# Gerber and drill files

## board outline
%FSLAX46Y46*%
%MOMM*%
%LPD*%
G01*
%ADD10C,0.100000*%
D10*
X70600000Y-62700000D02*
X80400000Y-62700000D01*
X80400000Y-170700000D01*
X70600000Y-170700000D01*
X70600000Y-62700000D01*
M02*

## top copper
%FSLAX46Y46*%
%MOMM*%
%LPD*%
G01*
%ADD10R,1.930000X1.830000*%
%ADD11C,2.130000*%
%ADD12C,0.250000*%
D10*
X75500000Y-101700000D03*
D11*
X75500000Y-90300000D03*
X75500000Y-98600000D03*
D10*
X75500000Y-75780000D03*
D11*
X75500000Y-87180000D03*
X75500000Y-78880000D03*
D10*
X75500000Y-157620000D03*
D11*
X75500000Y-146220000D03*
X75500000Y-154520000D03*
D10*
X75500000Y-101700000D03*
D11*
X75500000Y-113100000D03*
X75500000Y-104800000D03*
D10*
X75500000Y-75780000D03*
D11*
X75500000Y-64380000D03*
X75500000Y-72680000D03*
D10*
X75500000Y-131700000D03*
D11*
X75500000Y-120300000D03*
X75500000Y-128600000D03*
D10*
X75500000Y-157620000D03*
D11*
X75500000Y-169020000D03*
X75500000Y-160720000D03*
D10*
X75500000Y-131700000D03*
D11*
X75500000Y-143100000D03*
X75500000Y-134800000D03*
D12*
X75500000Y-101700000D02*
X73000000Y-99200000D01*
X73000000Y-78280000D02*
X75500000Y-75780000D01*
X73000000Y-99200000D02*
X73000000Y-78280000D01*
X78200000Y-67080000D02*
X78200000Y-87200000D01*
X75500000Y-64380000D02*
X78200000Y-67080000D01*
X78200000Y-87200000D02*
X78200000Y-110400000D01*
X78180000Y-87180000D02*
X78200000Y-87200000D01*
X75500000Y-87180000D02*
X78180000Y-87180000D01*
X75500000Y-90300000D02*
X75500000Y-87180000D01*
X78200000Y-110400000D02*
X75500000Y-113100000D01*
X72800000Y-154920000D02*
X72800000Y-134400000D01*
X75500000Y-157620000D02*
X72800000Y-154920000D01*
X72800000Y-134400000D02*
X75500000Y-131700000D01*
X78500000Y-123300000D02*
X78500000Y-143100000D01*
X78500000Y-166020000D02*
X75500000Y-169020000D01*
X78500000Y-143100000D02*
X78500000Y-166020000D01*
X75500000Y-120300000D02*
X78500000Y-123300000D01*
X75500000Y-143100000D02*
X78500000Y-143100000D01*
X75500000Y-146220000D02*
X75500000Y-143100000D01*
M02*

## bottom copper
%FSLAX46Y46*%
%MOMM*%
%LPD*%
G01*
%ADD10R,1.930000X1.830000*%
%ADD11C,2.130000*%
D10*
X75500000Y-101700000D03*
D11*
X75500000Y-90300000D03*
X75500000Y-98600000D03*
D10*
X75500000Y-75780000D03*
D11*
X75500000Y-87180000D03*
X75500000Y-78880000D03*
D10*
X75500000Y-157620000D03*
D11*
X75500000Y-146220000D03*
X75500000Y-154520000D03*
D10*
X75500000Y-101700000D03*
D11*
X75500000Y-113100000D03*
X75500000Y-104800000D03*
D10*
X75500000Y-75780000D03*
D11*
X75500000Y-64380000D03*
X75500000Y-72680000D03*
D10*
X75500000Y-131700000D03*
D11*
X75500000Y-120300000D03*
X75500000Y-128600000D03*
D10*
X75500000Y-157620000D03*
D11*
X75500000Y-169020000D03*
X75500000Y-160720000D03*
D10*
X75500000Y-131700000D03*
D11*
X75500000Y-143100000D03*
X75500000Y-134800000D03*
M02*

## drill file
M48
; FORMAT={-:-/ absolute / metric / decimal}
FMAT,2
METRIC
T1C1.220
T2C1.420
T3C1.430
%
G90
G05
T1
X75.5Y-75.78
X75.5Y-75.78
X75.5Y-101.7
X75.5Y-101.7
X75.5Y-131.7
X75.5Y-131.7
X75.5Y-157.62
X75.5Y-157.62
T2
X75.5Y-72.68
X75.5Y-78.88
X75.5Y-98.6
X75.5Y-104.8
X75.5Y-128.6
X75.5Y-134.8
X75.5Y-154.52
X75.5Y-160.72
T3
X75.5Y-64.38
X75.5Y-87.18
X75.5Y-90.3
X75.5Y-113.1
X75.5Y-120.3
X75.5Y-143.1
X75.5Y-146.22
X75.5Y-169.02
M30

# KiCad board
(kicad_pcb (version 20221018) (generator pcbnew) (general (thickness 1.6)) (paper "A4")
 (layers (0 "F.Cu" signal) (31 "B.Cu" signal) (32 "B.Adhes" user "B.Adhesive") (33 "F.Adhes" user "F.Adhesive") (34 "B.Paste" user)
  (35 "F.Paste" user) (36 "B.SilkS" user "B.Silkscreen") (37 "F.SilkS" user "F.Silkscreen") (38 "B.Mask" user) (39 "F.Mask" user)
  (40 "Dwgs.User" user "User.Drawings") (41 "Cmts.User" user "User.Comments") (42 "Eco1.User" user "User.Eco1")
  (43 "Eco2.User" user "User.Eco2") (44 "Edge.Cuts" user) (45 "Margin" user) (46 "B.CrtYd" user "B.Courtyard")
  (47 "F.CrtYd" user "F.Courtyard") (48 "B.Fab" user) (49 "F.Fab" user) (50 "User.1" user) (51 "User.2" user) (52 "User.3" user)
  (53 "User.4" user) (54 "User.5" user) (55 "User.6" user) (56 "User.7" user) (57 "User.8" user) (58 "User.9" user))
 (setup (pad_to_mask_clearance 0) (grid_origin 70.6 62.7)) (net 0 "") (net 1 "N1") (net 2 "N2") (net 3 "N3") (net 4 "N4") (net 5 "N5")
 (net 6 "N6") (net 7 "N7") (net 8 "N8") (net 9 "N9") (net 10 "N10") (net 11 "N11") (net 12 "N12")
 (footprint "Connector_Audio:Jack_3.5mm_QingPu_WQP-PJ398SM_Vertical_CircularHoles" (layer "F.Cu") (at 75.5 101.7 180)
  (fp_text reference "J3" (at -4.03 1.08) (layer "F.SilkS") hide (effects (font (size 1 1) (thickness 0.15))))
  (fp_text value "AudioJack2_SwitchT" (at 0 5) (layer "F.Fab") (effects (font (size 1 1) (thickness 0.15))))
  (pad "S" thru_hole rect (at 0 0) (size 1.93 1.83) (drill 1.22) (layers "*.Cu" "*.Mask") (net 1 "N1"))
  (pad "T" thru_hole circle (at 0 11.4) (size 2.13 2.13) (drill 1.43) (layers "*.Cu" "*.Mask") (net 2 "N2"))
  (pad "TN" thru_hole circle (at 0 3.1) (size 2.13 2.13) (drill 1.42) (layers "*.Cu" "*.Mask") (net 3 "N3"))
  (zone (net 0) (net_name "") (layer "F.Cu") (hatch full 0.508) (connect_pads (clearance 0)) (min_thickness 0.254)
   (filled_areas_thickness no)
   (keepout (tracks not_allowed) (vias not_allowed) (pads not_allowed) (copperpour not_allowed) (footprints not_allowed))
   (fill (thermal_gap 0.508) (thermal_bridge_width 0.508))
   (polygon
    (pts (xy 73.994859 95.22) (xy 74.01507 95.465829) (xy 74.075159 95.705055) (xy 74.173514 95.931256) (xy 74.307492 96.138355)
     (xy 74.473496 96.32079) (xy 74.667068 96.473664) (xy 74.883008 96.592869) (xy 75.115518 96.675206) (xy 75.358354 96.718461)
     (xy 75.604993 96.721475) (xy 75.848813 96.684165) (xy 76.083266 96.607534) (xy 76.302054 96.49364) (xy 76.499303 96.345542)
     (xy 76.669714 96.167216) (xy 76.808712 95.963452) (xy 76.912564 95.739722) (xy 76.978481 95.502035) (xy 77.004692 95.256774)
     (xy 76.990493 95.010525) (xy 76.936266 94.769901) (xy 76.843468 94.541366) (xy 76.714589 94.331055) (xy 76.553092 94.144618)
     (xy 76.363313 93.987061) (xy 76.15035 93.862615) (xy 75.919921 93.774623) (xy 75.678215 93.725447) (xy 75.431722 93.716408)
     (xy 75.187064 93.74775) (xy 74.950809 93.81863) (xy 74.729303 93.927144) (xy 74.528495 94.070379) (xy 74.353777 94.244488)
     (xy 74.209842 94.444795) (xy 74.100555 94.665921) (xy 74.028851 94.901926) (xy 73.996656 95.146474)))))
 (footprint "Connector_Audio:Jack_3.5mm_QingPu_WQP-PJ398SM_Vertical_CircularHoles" (layer "F.Cu") (at 75.5 75.78)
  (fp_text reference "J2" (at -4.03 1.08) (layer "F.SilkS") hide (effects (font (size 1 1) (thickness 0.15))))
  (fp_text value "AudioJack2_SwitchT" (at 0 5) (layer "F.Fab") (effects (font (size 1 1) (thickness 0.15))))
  (pad "S" thru_hole rect (at 0 0 180) (size 1.93 1.83) (drill 1.22) (layers "*.Cu" "*.Mask") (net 1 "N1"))
  (pad "T" thru_hole circle (at 0 11.4 180) (size 2.13 2.13) (drill 1.43) (layers "*.Cu" "*.Mask") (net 2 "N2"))
  (pad "TN" thru_hole circle (at 0 3.1 180) (size 2.13 2.13) (drill 1.42) (layers "*.Cu" "*.Mask") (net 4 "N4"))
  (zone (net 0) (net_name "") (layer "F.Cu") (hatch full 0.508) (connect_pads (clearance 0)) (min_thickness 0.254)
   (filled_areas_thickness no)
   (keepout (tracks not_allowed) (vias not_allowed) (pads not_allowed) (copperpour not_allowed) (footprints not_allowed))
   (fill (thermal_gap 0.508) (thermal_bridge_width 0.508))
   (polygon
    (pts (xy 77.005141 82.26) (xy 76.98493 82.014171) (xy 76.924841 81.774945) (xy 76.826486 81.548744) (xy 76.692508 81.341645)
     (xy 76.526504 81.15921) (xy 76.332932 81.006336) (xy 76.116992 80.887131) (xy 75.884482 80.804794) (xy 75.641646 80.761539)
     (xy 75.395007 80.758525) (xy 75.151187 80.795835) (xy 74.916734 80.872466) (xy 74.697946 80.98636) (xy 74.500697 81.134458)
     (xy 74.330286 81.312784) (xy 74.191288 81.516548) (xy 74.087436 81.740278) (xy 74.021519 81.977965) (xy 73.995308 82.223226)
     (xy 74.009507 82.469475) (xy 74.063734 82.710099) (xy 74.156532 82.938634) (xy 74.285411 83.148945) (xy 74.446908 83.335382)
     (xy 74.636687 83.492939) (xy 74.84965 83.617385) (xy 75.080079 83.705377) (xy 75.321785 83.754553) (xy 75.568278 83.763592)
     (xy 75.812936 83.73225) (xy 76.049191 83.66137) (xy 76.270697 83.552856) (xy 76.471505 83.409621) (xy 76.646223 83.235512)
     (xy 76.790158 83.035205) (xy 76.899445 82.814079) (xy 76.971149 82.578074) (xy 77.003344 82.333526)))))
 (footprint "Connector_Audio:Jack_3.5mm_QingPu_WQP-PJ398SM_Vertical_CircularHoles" (layer "F.Cu") (at 75.5 157.62 180)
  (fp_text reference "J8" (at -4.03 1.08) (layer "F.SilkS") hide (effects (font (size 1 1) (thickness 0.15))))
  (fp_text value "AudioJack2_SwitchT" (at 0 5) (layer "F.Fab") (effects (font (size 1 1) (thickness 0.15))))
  (pad "S" thru_hole rect (at 0 0) (size 1.93 1.83) (drill 1.22) (layers "*.Cu" "*.Mask") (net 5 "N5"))
  (pad "T" thru_hole circle (at 0 11.4) (size 2.13 2.13) (drill 1.43) (layers "*.Cu" "*.Mask") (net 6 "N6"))
  (pad "TN" thru_hole circle (at 0 3.1) (size 2.13 2.13) (drill 1.42) (layers "*.Cu" "*.Mask") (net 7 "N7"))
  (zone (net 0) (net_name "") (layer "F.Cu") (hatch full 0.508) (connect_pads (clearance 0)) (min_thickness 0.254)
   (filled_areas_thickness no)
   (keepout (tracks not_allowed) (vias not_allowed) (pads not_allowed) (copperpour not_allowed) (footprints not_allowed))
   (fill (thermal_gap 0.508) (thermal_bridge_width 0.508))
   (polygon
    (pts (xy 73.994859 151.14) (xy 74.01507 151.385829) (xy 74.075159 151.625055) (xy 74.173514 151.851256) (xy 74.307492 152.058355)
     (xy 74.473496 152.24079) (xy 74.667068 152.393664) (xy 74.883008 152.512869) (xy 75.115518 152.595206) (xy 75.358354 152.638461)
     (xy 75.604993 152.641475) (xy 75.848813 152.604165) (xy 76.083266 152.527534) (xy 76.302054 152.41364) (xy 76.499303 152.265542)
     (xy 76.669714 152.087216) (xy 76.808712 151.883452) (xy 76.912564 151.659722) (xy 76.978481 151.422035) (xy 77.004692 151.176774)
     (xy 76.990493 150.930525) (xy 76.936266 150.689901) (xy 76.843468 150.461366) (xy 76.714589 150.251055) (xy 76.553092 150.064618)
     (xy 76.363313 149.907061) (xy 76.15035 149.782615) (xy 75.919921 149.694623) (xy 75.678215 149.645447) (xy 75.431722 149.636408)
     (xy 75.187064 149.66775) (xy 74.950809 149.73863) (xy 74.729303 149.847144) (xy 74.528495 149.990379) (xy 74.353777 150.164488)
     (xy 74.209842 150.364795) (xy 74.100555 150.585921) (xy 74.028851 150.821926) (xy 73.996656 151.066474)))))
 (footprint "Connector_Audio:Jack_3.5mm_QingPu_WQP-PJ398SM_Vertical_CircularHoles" (layer "F.Cu") (at 75.5 101.7)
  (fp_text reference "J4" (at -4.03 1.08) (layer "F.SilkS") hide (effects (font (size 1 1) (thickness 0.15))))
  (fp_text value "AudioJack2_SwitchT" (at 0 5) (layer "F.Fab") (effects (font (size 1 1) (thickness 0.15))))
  (pad "S" thru_hole rect (at 0 0 180) (size 1.93 1.83) (drill 1.22) (layers "*.Cu" "*.Mask") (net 1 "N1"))
  (pad "T" thru_hole circle (at 0 11.4 180) (size 2.13 2.13) (drill 1.43) (layers "*.Cu" "*.Mask") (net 2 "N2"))
  (pad "TN" thru_hole circle (at 0 3.1 180) (size 2.13 2.13) (drill 1.42) (layers "*.Cu" "*.Mask") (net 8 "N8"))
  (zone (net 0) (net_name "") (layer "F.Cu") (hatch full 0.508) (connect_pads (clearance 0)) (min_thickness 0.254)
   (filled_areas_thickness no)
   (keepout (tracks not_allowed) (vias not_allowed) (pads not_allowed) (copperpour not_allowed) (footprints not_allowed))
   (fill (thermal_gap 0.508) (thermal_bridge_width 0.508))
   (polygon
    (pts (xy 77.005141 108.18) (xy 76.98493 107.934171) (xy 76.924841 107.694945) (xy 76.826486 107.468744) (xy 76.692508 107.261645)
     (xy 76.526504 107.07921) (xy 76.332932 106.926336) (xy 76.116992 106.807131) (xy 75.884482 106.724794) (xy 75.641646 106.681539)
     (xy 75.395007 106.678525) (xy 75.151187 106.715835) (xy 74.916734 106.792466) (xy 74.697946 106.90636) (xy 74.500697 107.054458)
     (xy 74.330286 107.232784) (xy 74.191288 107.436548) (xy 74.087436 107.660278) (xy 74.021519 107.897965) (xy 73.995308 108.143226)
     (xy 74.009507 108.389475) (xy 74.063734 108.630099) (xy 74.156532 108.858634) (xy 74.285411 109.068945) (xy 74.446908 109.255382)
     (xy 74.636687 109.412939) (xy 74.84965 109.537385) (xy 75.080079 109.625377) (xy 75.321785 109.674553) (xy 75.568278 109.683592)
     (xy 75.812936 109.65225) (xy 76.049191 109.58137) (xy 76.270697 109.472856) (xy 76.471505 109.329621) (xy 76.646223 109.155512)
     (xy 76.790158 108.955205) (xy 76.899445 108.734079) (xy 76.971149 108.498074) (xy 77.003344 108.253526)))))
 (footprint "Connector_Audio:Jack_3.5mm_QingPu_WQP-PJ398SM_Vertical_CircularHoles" (layer "F.Cu") (at 75.5 75.78 180)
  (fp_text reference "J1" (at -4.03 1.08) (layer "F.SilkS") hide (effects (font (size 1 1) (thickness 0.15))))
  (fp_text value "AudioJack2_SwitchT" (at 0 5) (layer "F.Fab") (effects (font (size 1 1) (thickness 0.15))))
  (pad "S" thru_hole rect (at 0 0) (size 1.93 1.83) (drill 1.22) (layers "*.Cu" "*.Mask") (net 1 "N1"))
  (pad "T" thru_hole circle (at 0 11.4) (size 2.13 2.13) (drill 1.43) (layers "*.Cu" "*.Mask") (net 2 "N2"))
  (pad "TN" thru_hole circle (at 0 3.1) (size 2.13 2.13) (drill 1.42) (layers "*.Cu" "*.Mask") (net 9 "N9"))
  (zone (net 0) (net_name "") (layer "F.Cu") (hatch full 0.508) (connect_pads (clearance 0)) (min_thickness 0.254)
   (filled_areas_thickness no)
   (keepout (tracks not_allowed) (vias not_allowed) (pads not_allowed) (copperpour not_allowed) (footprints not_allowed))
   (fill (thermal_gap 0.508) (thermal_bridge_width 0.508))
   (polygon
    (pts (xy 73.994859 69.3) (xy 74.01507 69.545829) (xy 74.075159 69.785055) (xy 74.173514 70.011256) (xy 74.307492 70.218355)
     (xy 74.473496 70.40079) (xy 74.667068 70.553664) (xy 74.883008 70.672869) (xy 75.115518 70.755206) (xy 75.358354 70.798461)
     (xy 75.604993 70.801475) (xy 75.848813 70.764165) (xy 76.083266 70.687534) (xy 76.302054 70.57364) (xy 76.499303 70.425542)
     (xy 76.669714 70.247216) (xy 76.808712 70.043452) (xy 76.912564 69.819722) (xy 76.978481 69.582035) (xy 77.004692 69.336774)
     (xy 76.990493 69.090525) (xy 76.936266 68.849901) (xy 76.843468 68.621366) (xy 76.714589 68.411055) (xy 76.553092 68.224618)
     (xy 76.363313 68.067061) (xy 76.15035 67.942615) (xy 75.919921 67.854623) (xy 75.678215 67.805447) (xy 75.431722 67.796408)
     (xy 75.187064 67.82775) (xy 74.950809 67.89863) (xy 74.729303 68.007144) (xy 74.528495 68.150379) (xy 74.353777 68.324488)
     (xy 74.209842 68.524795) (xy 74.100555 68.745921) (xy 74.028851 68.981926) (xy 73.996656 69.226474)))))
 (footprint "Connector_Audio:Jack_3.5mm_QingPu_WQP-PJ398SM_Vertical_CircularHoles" (layer "F.Cu") (at 75.5 131.7 180)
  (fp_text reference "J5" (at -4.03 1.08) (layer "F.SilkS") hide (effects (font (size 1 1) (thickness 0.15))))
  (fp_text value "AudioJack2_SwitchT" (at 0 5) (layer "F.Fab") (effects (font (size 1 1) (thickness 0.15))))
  (pad "S" thru_hole rect (at 0 0) (size 1.93 1.83) (drill 1.22) (layers "*.Cu" "*.Mask") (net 5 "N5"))
  (pad "T" thru_hole circle (at 0 11.4) (size 2.13 2.13) (drill 1.43) (layers "*.Cu" "*.Mask") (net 6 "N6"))
  (pad "TN" thru_hole circle (at 0 3.1) (size 2.13 2.13) (drill 1.42) (layers "*.Cu" "*.Mask") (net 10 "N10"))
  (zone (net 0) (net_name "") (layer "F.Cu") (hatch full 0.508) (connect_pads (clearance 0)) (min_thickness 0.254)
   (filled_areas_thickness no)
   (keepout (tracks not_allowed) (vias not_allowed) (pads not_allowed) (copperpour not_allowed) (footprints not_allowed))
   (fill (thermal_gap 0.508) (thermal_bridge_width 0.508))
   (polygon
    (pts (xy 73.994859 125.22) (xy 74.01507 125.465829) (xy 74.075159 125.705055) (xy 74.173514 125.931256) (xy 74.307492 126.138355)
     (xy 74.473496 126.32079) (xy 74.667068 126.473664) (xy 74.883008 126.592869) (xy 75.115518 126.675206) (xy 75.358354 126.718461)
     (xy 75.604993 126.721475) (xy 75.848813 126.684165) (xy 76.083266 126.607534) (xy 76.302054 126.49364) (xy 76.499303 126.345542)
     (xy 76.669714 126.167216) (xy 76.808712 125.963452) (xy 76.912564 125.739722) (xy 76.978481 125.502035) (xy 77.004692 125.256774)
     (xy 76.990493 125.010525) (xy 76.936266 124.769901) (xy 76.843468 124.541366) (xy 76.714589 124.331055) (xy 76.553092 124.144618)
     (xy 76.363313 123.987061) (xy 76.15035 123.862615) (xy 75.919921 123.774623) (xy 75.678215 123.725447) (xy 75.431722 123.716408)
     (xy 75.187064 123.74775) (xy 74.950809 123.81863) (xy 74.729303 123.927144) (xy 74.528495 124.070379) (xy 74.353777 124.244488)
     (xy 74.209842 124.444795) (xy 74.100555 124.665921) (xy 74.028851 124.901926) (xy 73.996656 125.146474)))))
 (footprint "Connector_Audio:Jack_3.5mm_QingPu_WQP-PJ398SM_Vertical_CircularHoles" (layer "F.Cu") (at 75.5 157.62)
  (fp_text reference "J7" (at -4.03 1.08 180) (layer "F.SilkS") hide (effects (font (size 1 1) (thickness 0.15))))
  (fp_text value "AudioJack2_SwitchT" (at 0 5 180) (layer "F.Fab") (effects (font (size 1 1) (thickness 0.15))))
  (pad "S" thru_hole rect (at 0 0 180) (size 1.93 1.83) (drill 1.22) (layers "*.Cu" "*.Mask") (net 5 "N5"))
  (pad "T" thru_hole circle (at 0 11.4 180) (size 2.13 2.13) (drill 1.43) (layers "*.Cu" "*.Mask") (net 6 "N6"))
  (pad "TN" thru_hole circle (at 0 3.1 180) (size 2.13 2.13) (drill 1.42) (layers "*.Cu" "*.Mask") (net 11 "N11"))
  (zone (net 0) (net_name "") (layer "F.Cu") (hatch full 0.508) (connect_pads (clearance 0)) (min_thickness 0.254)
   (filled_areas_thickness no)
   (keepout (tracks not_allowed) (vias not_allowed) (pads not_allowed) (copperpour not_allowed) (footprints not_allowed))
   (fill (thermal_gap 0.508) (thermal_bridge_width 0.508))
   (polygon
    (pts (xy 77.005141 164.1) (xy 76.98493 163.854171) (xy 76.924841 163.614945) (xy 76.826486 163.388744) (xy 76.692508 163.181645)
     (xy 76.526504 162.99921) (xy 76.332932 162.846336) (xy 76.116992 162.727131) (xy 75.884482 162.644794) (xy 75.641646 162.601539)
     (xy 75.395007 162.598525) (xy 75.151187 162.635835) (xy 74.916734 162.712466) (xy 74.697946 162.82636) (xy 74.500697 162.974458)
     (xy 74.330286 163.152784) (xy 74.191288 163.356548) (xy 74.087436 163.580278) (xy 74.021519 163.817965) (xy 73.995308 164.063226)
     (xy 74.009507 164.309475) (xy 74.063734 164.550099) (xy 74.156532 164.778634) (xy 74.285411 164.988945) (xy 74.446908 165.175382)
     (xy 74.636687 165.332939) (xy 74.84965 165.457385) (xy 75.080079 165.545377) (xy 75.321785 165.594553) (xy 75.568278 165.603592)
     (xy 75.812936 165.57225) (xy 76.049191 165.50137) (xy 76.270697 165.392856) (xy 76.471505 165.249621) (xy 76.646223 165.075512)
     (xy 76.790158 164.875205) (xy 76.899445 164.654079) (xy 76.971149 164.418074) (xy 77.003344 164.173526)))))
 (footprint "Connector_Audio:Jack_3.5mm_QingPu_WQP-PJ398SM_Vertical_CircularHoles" (layer "F.Cu") (at 75.5 131.7)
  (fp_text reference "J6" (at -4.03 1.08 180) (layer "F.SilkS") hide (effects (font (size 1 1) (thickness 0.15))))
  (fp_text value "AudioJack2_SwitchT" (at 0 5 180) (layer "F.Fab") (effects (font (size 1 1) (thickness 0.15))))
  (pad "S" thru_hole rect (at 0 0 180) (size 1.93 1.83) (drill 1.22) (layers "*.Cu" "*.Mask") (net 5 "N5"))
  (pad "T" thru_hole circle (at 0 11.4 180) (size 2.13 2.13) (drill 1.43) (layers "*.Cu" "*.Mask") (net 6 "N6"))
  (pad "TN" thru_hole circle (at 0 3.1 180) (size 2.13 2.13) (drill 1.42) (layers "*.Cu" "*.Mask") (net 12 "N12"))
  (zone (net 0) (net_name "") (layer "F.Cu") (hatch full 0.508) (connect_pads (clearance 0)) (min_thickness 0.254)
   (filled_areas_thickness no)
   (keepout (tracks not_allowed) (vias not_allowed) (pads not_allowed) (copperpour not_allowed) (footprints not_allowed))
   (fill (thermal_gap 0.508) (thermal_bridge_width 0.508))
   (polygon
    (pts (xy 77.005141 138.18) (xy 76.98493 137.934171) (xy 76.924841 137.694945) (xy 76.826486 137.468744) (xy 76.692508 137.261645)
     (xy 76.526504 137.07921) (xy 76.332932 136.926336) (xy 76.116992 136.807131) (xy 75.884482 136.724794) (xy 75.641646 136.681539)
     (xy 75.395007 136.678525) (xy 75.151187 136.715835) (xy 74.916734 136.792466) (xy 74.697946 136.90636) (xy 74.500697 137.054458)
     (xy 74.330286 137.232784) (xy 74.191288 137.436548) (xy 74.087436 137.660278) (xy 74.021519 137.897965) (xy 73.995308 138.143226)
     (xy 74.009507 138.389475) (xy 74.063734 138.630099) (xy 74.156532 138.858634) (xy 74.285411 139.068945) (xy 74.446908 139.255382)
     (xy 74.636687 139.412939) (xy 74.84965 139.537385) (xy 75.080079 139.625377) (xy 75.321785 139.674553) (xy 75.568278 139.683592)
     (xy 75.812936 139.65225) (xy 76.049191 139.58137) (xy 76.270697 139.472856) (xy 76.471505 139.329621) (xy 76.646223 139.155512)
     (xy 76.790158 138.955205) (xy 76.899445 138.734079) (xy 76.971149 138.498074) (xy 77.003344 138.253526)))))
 (gr_rect (start 70.6 62.7) (end 80.4 170.7) (stroke (width 0.1) (type default)) (fill none) (layer "Edge.Cuts"))
 (segment (start 75.5 101.7) (end 73 99.2) (width 0.25) (layer "F.Cu") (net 1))
 (segment (start 73 78.28) (end 75.5 75.78) (width 0.25) (layer "F.Cu") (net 1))
 (segment (start 73 99.2) (end 73 78.28) (width 0.25) (layer "F.Cu") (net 1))
 (segment (start 78.2 67.08) (end 78.2 87.2) (width 0.25) (layer "F.Cu") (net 2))
 (segment (start 75.5 64.38) (end 78.2 67.08) (width 0.25) (layer "F.Cu") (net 2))
 (segment (start 78.2 87.2) (end 78.2 110.4) (width 0.25) (layer "F.Cu") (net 2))
 (segment (start 78.18 87.18) (end 78.2 87.2) (width 0.25) (layer "F.Cu") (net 2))
 (segment (start 75.5 87.18) (end 78.18 87.18) (width 0.25) (layer "F.Cu") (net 2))
 (segment (start 75.5 90.3) (end 75.5 87.18) (width 0.25) (layer "F.Cu") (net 2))
 (segment (start 78.2 110.4) (end 75.5 113.1) (width 0.25) (layer "F.Cu") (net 2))
 (segment (start 72.8 154.92) (end 72.8 134.4) (width 0.25) (layer "F.Cu") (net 5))
 (segment (start 75.5 157.62) (end 72.8 154.92) (width 0.25) (layer "F.Cu") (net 5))
 (segment (start 72.8 134.4) (end 75.5 131.7) (width 0.25) (layer "F.Cu") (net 5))
 (segment (start 78.5 123.3) (end 78.5 143.1) (width 0.25) (layer "F.Cu") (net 6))
 (segment (start 78.5 166.02) (end 75.5 169.02) (width 0.25) (layer "F.Cu") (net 6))
 (segment (start 78.5 143.1) (end 78.5 166.02) (width 0.25) (layer "F.Cu") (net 6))
 (segment (start 75.5 120.3) (end 78.5 123.3) (width 0.25) (layer "F.Cu") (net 6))
 (segment (start 75.5 143.1) (end 78.5 143.1) (width 0.25) (layer "F.Cu") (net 6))
 (segment (start 75.5 146.22) (end 75.5 143.1) (width 0.25) (layer "F.Cu") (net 6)))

